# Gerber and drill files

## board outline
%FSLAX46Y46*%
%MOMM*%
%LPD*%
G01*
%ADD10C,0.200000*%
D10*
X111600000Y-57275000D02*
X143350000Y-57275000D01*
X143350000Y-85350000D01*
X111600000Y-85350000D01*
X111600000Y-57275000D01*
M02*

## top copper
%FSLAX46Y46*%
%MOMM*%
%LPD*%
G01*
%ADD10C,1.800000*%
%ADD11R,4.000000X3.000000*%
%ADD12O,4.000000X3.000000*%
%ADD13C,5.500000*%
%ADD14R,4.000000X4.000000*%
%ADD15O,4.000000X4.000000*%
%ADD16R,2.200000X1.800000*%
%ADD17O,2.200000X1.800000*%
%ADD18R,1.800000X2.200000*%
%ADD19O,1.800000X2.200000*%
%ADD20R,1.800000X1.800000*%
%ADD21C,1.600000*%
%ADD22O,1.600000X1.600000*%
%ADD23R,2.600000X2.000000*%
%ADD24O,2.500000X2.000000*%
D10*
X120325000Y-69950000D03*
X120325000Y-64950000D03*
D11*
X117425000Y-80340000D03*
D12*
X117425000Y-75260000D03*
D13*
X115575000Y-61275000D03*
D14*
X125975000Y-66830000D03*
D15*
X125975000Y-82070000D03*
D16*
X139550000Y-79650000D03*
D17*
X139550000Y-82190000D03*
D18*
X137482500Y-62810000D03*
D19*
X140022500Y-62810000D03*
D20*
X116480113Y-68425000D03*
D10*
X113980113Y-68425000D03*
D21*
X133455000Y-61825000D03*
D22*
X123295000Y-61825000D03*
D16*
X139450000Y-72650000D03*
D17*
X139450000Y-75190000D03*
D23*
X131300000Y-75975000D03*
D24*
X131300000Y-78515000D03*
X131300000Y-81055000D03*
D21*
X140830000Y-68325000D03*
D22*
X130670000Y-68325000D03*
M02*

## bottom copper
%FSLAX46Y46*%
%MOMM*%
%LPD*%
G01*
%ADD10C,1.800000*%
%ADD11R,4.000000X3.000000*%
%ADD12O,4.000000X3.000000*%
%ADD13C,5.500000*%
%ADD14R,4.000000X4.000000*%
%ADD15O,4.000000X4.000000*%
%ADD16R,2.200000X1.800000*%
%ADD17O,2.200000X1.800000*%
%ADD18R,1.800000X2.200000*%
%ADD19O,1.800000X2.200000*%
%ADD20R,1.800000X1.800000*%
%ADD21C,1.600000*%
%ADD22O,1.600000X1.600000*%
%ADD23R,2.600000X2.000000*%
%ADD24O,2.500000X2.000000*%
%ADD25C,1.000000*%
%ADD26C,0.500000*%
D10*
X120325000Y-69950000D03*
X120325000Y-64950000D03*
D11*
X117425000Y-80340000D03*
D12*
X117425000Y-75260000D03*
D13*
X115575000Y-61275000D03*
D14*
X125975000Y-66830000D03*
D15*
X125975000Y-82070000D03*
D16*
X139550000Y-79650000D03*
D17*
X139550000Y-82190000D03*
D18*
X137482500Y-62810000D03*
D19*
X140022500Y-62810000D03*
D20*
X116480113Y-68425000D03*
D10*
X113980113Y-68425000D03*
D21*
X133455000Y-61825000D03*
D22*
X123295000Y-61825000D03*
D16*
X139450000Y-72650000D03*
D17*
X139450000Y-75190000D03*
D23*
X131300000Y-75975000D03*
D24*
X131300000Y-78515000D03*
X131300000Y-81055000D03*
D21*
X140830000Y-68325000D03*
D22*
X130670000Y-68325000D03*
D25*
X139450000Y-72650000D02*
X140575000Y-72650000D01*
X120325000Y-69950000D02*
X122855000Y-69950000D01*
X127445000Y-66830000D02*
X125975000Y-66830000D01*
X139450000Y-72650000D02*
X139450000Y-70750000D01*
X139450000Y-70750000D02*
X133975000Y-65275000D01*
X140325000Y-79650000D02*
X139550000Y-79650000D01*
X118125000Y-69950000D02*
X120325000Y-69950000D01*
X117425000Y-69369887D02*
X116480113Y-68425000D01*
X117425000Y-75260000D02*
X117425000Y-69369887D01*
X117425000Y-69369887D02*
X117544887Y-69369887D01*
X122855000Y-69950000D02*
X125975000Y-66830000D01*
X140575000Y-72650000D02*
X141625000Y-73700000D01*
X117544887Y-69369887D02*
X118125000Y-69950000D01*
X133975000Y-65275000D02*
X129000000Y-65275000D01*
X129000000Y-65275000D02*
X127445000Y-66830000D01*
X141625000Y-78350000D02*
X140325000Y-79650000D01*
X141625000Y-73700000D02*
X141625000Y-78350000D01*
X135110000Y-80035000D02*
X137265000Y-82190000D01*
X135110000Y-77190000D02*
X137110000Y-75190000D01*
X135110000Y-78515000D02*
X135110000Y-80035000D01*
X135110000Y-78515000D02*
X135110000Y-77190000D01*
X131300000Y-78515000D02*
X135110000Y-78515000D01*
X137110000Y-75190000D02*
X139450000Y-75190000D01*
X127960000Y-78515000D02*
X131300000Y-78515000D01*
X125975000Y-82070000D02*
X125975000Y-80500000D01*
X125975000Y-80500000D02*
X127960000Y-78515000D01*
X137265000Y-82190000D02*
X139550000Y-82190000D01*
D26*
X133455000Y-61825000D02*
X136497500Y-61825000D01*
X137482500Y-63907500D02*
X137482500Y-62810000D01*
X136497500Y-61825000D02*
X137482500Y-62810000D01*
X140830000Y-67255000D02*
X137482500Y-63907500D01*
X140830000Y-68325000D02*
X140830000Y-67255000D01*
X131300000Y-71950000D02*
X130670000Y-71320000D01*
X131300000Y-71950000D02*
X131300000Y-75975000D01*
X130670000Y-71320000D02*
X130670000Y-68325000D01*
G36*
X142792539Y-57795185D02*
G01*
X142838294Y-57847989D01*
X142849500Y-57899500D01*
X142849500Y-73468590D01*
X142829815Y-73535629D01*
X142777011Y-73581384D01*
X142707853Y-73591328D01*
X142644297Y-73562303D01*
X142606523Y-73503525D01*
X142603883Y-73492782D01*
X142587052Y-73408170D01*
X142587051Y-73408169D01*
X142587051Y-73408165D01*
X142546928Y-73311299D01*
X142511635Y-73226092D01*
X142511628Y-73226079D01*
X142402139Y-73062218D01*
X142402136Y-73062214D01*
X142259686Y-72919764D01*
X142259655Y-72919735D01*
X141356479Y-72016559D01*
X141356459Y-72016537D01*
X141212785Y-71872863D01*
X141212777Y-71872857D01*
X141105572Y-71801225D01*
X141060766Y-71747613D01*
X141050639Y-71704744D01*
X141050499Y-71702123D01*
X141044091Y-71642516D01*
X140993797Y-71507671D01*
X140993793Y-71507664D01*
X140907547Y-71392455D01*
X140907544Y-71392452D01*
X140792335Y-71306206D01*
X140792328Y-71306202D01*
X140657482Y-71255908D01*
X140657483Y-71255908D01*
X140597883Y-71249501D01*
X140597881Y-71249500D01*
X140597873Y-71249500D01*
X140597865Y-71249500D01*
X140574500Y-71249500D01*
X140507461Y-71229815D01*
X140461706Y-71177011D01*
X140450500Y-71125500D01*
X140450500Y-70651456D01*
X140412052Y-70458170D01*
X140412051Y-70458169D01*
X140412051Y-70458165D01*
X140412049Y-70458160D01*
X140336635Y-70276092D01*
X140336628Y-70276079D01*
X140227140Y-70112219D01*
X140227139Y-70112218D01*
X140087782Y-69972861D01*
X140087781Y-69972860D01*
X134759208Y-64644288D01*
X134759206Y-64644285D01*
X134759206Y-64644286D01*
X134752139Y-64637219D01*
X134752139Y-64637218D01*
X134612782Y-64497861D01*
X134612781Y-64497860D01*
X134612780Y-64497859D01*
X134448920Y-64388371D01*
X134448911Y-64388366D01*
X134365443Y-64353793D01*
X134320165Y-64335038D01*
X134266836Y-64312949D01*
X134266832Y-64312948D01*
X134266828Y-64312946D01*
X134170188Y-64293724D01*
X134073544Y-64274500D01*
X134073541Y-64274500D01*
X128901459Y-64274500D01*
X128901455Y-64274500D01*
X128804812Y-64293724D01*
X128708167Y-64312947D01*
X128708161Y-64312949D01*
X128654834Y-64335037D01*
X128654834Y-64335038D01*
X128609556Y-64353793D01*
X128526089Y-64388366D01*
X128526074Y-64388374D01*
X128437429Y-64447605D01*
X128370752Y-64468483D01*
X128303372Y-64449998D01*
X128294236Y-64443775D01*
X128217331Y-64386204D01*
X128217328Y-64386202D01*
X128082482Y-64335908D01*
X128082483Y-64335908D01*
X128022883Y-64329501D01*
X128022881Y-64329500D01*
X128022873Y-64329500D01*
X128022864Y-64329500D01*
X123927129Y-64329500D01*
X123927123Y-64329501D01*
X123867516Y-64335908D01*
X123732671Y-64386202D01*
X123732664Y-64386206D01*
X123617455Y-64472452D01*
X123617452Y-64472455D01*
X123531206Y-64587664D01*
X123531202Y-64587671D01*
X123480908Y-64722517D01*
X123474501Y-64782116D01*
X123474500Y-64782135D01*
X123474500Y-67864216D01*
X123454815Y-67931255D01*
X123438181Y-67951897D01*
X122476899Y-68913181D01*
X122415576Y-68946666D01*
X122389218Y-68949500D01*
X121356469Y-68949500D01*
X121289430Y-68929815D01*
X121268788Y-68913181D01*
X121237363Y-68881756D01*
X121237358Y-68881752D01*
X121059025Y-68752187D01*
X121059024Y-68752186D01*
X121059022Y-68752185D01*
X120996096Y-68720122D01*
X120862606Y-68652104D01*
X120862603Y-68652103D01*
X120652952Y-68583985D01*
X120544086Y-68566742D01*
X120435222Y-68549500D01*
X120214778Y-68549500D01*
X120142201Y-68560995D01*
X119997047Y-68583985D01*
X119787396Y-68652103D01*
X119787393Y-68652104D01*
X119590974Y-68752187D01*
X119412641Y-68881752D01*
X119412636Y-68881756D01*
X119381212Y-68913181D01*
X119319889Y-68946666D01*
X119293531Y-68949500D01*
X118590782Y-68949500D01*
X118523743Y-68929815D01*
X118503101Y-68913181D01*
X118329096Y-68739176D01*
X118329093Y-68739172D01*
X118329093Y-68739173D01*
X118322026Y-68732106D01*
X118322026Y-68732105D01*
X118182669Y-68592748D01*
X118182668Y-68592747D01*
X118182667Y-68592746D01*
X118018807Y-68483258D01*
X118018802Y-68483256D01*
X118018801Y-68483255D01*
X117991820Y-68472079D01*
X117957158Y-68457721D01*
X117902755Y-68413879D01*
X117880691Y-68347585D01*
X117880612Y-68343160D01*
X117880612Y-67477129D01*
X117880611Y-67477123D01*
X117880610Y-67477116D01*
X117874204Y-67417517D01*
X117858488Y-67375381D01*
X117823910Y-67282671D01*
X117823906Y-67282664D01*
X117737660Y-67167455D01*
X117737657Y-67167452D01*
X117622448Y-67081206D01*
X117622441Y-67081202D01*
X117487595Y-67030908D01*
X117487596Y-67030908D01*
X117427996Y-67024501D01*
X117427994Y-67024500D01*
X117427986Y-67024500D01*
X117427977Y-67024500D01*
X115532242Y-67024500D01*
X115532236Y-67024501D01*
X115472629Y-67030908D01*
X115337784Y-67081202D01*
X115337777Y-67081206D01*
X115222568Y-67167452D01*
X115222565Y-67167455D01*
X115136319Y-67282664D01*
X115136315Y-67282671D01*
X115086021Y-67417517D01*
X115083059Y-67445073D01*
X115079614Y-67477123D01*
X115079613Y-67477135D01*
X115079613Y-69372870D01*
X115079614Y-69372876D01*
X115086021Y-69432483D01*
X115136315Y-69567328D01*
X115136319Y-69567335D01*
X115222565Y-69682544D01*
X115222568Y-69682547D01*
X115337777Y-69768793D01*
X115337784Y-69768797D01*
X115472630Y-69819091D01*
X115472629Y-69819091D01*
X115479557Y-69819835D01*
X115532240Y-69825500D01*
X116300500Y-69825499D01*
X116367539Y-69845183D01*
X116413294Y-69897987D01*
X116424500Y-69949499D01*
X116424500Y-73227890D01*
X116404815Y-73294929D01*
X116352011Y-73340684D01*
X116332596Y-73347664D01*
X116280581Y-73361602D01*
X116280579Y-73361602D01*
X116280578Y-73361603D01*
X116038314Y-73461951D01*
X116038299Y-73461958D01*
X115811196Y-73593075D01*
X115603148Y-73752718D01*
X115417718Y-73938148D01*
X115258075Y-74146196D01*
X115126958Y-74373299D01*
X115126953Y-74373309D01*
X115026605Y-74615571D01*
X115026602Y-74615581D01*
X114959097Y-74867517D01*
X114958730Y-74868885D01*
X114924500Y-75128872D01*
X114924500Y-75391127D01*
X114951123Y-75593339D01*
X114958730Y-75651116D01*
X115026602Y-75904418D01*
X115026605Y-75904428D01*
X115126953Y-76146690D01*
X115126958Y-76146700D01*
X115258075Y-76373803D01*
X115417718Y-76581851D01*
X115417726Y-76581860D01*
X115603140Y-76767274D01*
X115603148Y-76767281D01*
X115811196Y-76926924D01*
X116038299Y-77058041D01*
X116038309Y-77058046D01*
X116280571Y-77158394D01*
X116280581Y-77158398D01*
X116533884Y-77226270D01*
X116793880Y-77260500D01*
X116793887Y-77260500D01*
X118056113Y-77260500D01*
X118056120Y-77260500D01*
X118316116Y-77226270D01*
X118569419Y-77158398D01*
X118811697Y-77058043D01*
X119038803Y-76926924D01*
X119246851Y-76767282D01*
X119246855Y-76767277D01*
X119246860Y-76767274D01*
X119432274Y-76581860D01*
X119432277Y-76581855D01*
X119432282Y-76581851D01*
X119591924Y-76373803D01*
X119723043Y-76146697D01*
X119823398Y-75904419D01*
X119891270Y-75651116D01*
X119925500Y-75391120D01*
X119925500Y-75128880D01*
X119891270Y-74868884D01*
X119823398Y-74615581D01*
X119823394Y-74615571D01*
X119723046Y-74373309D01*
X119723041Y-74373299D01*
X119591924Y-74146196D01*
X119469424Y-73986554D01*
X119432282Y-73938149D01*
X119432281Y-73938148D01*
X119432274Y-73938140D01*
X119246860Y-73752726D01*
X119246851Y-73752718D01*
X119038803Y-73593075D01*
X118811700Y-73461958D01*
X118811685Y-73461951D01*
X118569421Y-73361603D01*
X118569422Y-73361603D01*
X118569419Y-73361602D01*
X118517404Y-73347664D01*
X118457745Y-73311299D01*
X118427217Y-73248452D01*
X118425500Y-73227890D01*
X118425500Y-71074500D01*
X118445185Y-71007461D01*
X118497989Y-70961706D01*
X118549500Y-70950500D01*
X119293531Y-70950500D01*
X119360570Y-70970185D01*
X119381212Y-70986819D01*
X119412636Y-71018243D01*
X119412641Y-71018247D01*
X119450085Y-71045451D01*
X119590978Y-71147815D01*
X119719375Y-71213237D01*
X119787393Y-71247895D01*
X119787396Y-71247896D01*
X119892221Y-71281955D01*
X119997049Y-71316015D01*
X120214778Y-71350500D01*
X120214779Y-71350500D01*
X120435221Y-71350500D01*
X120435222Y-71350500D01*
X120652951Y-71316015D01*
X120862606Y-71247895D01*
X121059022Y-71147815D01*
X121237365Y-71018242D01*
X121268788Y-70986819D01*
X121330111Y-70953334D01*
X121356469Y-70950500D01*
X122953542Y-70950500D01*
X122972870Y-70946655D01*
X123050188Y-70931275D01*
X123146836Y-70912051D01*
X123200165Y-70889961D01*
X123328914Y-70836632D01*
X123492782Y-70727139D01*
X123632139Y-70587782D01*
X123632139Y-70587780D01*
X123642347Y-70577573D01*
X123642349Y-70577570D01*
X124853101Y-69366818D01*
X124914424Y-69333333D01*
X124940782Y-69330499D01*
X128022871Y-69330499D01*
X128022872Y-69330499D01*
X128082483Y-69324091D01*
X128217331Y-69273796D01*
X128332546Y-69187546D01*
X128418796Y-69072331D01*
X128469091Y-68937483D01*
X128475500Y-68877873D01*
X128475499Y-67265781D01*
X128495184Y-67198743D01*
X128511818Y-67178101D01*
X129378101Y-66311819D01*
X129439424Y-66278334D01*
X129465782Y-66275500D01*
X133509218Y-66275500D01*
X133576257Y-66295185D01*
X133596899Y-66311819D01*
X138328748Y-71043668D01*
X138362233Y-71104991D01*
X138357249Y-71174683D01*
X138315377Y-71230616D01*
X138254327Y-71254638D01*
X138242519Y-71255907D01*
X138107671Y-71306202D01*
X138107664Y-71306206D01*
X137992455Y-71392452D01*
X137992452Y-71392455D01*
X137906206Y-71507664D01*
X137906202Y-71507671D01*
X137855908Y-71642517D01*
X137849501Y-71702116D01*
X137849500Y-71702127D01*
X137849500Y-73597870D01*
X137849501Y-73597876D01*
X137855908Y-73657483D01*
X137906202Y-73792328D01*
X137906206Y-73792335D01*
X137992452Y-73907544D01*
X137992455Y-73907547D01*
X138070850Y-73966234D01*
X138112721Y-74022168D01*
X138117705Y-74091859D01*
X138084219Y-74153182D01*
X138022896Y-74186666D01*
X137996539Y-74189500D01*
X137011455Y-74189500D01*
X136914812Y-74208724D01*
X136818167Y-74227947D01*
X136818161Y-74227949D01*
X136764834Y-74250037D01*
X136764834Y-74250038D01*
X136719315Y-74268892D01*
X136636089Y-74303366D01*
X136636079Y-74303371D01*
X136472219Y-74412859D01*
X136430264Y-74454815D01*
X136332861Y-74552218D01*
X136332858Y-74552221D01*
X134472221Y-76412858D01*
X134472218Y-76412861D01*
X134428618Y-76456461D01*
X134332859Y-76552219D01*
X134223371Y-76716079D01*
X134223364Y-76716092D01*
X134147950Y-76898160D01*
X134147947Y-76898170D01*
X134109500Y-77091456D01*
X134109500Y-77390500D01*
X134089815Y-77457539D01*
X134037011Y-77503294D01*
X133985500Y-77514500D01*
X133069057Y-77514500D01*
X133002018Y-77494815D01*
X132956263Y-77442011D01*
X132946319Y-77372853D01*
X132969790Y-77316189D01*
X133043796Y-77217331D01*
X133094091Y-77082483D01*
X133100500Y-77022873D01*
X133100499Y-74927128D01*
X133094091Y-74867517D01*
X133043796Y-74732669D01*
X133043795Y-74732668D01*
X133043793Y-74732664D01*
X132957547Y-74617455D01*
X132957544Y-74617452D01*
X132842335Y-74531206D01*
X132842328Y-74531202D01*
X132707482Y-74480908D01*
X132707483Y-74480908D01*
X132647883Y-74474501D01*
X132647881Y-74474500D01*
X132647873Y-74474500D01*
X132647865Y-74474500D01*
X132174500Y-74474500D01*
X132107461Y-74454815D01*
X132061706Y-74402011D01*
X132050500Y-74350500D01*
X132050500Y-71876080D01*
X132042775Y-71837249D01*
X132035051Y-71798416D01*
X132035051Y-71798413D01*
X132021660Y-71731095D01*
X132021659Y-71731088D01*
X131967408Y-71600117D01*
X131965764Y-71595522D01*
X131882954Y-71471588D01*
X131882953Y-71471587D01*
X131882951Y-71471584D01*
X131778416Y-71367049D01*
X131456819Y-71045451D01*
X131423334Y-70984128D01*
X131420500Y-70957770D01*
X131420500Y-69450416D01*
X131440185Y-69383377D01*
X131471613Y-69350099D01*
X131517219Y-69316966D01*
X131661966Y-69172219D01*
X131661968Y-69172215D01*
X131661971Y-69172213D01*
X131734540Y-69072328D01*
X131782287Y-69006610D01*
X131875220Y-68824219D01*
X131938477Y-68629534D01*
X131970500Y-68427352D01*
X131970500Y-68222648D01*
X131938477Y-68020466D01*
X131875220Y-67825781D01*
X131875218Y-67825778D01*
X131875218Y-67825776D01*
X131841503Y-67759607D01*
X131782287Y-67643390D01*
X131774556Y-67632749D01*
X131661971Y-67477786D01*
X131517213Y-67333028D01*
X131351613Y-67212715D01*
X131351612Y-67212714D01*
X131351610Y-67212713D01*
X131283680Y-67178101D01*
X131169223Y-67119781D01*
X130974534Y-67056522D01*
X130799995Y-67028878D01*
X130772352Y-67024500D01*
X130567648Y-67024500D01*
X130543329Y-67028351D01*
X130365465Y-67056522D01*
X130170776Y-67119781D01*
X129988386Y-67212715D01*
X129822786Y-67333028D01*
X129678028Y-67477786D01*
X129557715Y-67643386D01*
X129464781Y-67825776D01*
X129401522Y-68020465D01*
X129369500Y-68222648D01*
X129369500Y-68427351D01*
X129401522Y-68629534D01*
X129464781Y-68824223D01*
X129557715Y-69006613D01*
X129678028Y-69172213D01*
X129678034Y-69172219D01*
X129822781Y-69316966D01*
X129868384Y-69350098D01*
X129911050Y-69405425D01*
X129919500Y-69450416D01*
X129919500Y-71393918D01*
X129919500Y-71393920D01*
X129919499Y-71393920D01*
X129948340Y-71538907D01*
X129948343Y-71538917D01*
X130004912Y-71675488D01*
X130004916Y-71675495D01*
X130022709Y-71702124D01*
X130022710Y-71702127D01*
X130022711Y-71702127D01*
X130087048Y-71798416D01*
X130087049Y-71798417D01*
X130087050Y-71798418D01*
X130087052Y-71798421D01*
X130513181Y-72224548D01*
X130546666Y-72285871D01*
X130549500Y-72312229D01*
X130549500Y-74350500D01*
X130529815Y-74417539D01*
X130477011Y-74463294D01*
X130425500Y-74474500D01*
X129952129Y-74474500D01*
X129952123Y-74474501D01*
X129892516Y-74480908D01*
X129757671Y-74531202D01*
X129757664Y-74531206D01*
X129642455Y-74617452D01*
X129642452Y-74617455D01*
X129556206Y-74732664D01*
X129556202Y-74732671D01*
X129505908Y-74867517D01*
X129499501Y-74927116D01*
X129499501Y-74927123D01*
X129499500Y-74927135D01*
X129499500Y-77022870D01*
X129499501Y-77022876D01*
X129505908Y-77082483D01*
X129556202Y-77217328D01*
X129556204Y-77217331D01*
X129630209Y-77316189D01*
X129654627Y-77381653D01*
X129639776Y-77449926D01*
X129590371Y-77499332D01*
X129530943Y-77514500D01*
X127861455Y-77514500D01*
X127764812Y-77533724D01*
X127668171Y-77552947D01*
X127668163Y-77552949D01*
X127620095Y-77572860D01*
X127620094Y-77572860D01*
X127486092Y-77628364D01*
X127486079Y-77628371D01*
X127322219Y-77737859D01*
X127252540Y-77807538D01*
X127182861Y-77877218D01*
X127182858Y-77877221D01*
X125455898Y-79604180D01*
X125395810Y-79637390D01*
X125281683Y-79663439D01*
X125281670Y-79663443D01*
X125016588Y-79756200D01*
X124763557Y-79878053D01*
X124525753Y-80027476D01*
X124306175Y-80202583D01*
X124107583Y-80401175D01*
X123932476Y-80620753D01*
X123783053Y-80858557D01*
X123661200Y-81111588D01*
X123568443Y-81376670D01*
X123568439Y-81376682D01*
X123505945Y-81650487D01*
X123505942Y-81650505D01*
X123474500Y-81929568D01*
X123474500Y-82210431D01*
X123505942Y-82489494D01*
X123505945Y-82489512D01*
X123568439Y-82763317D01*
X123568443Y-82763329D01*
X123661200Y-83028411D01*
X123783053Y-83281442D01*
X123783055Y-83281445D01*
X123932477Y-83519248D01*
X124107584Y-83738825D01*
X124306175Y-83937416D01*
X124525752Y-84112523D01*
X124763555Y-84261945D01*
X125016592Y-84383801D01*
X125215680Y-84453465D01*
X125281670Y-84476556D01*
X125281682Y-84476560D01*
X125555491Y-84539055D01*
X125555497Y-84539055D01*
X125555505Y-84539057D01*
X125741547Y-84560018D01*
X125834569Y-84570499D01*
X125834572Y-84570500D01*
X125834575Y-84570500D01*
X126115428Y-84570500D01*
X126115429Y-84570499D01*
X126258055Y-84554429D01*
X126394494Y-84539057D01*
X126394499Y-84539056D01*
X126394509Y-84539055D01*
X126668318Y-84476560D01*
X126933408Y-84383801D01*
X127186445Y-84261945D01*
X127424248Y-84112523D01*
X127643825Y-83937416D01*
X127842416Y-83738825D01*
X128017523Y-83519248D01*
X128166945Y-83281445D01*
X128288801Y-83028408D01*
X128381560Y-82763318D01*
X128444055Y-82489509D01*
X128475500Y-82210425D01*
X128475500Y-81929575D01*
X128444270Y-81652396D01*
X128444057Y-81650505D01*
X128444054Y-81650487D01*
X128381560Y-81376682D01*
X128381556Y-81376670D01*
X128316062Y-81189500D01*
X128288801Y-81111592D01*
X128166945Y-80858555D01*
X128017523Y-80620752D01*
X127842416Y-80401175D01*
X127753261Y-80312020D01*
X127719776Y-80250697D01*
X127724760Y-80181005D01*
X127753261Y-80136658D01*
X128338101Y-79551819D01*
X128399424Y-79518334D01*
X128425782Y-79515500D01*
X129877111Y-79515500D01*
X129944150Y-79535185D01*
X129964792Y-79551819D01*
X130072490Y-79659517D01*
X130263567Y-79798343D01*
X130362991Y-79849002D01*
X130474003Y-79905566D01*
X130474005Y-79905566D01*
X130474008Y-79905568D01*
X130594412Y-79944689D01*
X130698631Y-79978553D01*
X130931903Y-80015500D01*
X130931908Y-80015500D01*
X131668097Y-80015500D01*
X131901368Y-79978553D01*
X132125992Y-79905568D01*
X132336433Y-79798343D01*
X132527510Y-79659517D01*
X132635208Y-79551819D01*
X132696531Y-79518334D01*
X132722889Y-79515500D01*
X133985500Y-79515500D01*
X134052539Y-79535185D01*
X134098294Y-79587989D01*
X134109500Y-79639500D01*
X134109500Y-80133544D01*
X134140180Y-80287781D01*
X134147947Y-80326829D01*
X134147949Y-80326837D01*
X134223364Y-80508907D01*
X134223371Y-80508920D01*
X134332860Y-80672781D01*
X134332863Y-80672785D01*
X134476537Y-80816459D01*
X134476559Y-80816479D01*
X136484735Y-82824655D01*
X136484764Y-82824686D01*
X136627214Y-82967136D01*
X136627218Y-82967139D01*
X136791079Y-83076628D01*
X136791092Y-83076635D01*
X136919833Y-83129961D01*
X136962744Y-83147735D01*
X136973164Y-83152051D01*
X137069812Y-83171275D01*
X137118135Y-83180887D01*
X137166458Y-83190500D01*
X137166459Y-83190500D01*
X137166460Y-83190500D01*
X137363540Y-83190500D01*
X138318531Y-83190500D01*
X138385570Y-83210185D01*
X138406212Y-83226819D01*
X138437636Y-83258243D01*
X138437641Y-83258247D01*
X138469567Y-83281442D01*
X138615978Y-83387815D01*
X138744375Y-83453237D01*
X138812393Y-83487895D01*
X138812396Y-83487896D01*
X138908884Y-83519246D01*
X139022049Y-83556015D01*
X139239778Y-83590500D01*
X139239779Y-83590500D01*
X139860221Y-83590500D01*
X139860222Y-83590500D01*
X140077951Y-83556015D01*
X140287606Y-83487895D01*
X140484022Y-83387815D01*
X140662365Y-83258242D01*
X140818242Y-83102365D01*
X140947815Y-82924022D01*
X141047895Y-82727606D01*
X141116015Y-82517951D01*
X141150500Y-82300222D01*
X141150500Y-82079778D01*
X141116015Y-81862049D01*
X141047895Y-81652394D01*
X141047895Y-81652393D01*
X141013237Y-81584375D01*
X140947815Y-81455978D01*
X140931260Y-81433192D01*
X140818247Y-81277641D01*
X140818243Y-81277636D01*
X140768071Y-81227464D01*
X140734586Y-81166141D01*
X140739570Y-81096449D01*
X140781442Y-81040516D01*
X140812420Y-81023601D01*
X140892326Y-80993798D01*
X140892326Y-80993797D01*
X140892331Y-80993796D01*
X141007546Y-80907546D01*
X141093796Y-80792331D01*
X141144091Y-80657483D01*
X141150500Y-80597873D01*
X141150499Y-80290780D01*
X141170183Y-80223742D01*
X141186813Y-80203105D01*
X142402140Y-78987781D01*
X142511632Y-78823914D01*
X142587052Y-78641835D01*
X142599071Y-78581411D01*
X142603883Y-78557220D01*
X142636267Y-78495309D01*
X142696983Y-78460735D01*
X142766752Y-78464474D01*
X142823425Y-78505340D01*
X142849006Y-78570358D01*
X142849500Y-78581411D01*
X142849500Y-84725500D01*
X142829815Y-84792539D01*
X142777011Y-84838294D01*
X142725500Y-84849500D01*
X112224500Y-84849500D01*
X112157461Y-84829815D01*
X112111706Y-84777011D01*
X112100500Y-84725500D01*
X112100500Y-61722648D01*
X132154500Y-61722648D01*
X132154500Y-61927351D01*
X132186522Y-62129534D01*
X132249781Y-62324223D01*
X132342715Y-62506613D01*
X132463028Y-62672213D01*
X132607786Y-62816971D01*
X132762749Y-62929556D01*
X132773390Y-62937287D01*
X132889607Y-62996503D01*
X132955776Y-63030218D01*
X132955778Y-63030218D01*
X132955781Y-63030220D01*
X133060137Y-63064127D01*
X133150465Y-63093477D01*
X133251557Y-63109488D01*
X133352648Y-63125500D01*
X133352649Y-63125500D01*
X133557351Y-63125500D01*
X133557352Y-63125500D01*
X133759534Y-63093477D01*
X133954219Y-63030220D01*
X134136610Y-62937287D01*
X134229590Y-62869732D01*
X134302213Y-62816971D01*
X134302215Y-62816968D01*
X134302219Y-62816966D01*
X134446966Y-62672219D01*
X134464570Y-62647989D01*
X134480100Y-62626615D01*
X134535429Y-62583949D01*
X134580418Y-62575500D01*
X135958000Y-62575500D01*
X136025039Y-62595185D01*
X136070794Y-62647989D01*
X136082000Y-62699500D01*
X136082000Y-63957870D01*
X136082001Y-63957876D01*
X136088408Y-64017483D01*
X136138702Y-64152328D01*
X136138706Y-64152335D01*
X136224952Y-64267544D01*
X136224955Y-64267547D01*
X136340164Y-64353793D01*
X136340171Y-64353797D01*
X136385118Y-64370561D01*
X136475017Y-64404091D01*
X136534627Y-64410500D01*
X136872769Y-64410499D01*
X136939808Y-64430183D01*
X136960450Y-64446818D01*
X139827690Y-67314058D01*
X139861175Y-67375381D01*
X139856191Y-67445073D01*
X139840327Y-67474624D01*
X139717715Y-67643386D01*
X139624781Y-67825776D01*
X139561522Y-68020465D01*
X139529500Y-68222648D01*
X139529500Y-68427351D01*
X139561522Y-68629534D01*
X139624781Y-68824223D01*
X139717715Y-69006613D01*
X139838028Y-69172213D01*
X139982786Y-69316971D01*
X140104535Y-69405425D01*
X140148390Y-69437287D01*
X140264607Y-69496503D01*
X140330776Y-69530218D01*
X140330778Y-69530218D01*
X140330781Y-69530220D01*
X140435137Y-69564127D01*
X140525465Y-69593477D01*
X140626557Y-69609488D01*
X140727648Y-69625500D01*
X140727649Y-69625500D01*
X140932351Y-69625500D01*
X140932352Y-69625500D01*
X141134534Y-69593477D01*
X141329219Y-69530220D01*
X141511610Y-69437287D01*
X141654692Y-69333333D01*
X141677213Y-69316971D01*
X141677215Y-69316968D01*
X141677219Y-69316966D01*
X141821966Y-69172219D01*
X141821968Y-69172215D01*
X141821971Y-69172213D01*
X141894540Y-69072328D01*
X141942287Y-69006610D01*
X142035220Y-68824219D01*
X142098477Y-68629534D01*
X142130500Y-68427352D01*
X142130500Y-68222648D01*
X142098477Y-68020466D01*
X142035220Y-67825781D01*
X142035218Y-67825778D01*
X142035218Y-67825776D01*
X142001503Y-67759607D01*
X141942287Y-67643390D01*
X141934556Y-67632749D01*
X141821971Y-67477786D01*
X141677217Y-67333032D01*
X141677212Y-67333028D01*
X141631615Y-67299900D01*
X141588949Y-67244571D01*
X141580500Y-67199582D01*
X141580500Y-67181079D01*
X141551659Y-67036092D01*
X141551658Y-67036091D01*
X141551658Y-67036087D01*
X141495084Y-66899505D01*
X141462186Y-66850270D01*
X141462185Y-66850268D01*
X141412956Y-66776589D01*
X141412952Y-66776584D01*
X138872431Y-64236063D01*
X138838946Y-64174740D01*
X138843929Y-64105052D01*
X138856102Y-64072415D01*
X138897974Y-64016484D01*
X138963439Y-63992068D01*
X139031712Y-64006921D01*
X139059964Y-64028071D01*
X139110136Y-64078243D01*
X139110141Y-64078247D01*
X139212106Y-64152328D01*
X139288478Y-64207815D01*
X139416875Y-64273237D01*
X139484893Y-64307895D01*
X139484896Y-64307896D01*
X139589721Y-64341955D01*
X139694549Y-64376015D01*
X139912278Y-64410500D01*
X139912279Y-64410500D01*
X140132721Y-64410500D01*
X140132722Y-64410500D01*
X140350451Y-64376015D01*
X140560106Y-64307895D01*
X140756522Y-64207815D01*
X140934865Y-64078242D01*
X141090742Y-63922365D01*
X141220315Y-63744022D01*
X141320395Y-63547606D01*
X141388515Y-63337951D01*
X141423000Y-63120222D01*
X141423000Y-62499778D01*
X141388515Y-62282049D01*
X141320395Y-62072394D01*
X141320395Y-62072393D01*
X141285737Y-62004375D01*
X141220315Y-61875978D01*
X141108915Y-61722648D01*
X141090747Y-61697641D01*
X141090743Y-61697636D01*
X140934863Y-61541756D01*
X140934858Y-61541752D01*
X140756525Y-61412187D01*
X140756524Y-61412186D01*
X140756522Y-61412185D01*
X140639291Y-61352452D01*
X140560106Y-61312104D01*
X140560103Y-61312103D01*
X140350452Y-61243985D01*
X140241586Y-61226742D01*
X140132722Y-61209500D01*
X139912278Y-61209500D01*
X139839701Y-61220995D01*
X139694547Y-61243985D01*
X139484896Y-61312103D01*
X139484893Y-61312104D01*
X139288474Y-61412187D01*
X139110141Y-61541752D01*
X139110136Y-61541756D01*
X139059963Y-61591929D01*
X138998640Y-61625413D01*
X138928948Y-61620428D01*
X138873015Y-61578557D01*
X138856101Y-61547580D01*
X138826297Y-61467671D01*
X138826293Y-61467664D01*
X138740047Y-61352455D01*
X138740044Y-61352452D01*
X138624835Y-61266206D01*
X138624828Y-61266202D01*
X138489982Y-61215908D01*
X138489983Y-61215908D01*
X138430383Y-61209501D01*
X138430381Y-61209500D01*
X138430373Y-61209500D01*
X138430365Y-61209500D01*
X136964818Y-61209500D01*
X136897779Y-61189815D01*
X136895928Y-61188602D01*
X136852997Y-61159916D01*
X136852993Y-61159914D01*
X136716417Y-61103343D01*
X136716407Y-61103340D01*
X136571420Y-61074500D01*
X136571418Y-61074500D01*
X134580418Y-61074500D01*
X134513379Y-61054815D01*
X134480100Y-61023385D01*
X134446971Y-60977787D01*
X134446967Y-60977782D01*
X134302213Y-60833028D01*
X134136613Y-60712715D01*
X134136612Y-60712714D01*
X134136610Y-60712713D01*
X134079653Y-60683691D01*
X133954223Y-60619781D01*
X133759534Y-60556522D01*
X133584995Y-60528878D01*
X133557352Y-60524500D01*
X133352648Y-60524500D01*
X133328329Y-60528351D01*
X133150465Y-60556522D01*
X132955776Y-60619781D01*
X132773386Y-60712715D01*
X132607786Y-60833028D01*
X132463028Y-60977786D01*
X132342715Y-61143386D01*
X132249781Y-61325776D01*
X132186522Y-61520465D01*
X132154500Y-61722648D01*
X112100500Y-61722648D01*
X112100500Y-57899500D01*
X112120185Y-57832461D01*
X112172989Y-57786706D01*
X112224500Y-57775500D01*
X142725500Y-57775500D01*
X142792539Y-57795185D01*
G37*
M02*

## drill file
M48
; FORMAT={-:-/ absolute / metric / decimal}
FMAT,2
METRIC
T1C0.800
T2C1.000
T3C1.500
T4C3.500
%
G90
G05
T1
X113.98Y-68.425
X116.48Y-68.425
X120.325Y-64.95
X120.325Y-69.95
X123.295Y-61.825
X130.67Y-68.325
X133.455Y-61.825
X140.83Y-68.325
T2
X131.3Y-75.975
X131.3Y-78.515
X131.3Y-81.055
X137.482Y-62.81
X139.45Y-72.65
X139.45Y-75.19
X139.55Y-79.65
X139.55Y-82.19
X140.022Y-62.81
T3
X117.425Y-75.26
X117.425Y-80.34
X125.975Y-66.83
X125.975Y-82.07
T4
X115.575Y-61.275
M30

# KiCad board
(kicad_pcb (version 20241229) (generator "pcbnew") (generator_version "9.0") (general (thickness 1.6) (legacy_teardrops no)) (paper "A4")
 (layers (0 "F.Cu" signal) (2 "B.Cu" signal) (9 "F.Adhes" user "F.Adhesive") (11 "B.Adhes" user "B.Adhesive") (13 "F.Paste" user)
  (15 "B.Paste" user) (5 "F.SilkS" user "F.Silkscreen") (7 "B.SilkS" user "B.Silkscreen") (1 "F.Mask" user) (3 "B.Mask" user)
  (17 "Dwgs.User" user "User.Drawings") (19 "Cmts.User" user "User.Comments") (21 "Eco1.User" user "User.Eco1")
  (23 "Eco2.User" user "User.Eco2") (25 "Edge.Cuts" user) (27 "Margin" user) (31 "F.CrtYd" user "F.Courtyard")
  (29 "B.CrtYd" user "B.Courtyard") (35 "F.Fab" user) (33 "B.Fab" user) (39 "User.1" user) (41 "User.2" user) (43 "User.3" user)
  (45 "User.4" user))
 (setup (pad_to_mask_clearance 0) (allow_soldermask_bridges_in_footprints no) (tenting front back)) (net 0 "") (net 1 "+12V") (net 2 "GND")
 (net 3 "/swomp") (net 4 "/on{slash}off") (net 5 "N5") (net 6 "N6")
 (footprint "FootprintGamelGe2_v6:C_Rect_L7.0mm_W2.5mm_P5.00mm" (layer "F.Cu") (at 120.325 69.95 90)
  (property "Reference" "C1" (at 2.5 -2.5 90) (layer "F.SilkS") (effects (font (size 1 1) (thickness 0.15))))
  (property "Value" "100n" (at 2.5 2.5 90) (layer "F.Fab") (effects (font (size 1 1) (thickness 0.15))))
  (pad "1" thru_hole circle (at 0 0 90) (size 1.8 1.8) (drill 0.8) (layers "*.Cu" "*.Mask") (remove_unused_layers no) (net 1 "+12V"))
  (pad "2" thru_hole circle (at 5 0 90) (size 1.8 1.8) (drill 0.8) (layers "*.Cu" "*.Mask") (remove_unused_layers no) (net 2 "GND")))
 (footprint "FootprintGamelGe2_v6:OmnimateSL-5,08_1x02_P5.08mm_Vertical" (layer "F.Cu") (at 117.425 80.34 90)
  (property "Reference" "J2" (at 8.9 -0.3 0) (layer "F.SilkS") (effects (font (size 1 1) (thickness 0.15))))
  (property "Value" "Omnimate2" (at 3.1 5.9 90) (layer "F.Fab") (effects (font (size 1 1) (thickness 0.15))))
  (pad "1" thru_hole rect (at 0 0 90) (size 3 4) (drill 1.5) (layers "*.Cu" "*.Mask") (remove_unused_layers no) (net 2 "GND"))
  (pad "2" thru_hole oval (at 5.08 0 90) (size 3 4) (drill 1.5) (layers "*.Cu" "*.Mask") (remove_unused_layers no) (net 1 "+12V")))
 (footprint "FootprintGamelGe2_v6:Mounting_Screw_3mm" (layer "F.Cu") (at 115.575 61.275)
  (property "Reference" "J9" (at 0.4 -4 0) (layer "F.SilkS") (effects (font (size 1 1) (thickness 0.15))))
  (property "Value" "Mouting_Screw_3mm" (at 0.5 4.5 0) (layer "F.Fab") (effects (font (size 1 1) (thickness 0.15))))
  (pad "1" thru_hole circle (at 0 0) (size 5.5 5.5) (drill 3.5) (layers "*.Cu" "*.Mask") (remove_unused_layers no) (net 2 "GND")))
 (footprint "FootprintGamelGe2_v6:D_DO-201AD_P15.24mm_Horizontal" (layer "F.Cu") (at 125.975 66.83 -90)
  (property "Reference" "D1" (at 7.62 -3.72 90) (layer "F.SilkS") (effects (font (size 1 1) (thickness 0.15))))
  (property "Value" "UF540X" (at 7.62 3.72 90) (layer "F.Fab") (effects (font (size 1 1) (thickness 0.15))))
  (pad "1" thru_hole rect (at 0 0 270) (size 4 4) (drill 1.5) (layers "*.Cu" "*.Mask") (remove_unused_layers no) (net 1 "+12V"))
  (pad "2" thru_hole oval (at 15.24 0 270) (size 4 4) (drill 1.5) (layers "*.Cu" "*.Mask") (remove_unused_layers no) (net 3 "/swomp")))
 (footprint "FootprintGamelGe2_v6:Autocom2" (layer "F.Cu") (at 139.55 79.65)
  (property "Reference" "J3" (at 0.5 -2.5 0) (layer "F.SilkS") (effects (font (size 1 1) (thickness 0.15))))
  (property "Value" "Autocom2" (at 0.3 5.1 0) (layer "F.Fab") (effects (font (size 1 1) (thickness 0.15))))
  (pad "1" thru_hole rect (at 0 0) (size 2.2 1.8) (drill 1) (layers "*.Cu" "*.Mask") (remove_unused_layers no) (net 1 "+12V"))
  (pad "2" thru_hole oval (at 0 2.54) (size 2.2 1.8) (drill 1) (layers "*.Cu" "*.Mask") (remove_unused_layers no) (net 3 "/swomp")))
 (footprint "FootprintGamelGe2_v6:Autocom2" (layer "F.Cu") (at 137.4825 62.81 90)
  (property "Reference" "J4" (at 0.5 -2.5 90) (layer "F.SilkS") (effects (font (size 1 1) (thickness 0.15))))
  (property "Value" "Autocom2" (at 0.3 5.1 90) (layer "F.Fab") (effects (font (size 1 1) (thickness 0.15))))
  (pad "1" thru_hole rect (at 0 0 90) (size 2.2 1.8) (drill 1) (layers "*.Cu" "*.Mask") (remove_unused_layers no) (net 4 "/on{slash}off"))
  (pad "2" thru_hole oval (at 0 2.54 90) (size 2.2 1.8) (drill 1) (layers "*.Cu" "*.Mask") (remove_unused_layers no) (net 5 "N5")))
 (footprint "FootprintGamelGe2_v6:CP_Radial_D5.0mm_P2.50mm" (layer "F.Cu") (at 116.480113 68.425 180)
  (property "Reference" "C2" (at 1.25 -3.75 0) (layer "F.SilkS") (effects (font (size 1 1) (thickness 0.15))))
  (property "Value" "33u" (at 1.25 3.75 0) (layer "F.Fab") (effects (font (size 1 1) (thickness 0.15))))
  (pad "1" thru_hole rect (at 0 0 180) (size 1.8 1.8) (drill 0.8) (layers "*.Cu" "*.Mask") (remove_unused_layers no) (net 1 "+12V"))
  (pad "2" thru_hole circle (at 2.5 0 180) (size 1.8 1.8) (drill 0.8) (layers "*.Cu" "*.Mask") (remove_unused_layers no) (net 2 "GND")))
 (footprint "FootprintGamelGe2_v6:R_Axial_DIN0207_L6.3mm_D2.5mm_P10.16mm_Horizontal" (layer "F.Cu") (at 133.455 61.825 180)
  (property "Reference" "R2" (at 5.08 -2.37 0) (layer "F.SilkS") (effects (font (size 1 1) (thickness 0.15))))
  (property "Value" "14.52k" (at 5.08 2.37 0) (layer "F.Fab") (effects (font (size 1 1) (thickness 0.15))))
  (pad "1" thru_hole circle (at 0 0 180) (size 1.6 1.6) (drill 0.8) (layers "*.Cu" "*.Mask") (remove_unused_layers no)
   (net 4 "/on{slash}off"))
  (pad "2" thru_hole oval (at 10.16 0 180) (size 1.6 1.6) (drill 0.8) (layers "*.Cu" "*.Mask") (remove_unused_layers no) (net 2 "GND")))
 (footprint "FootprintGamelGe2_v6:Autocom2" (layer "F.Cu") (at 139.45 72.65)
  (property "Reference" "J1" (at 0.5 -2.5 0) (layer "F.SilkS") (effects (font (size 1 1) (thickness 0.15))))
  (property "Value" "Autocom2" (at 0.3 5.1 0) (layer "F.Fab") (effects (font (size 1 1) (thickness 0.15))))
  (pad "1" thru_hole rect (at 0 0) (size 2.2 1.8) (drill 1) (layers "*.Cu" "*.Mask") (remove_unused_layers no) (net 1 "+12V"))
  (pad "2" thru_hole oval (at 0 2.54) (size 2.2 1.8) (drill 1) (layers "*.Cu" "*.Mask") (remove_unused_layers no) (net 3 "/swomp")))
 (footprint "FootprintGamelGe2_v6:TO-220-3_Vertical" (layer "F.Cu") (at 131.3 75.975 -90)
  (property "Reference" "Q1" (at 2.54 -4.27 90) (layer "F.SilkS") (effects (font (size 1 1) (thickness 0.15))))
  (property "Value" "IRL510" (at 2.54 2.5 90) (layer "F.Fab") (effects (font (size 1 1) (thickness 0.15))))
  (pad "1" thru_hole rect (at 0 0 270) (size 2 2.6) (drill 1) (layers "*.Cu" "*.Mask") (remove_unused_layers no) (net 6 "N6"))
  (pad "2" thru_hole oval (at 2.54 0 270) (size 2 2.5) (drill 1) (layers "*.Cu" "*.Mask") (remove_unused_layers no) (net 3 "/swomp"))
  (pad "3" thru_hole oval (at 5.08 0 270) (size 2 2.5) (drill 1) (layers "*.Cu" "*.Mask") (remove_unused_layers no) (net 2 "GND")))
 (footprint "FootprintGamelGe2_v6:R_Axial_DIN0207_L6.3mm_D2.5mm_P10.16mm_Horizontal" (layer "F.Cu") (at 140.83 68.325 180)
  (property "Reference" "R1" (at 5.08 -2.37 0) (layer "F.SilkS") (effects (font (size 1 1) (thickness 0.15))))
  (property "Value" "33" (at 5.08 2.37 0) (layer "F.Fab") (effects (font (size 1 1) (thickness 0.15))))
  (pad "1" thru_hole circle (at 0 0 180) (size 1.6 1.6) (drill 0.8) (layers "*.Cu" "*.Mask") (remove_unused_layers no)
   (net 4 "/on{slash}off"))
  (pad "2" thru_hole oval (at 10.16 0 180) (size 1.6 1.6) (drill 0.8) (layers "*.Cu" "*.Mask") (remove_unused_layers no) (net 6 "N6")))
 (gr_rect (start 111.6 57.275) (end 143.35 85.35) (stroke (width 0.2) (type solid)) (fill no) (layer "Edge.Cuts"))
 (segment (start 139.45 72.65) (end 140.575 72.65) (width 1) (layer "B.Cu") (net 1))
 (segment (start 120.325 69.95) (end 122.855 69.95) (width 1) (layer "B.Cu") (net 1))
 (segment (start 127.445 66.83) (end 125.975 66.83) (width 1) (layer "B.Cu") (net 1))
 (segment (start 139.45 72.65) (end 139.45 70.75) (width 1) (layer "B.Cu") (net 1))
 (segment (start 139.45 70.75) (end 133.975 65.275) (width 1) (layer "B.Cu") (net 1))
 (segment (start 140.325 79.65) (end 139.55 79.65) (width 1) (layer "B.Cu") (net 1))
 (segment (start 118.125 69.95) (end 120.325 69.95) (width 1) (layer "B.Cu") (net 1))
 (segment (start 117.425 69.369887) (end 116.480113 68.425) (width 1) (layer "B.Cu") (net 1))
 (segment (start 117.425 75.26) (end 117.425 69.369887) (width 1) (layer "B.Cu") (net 1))
 (segment (start 117.425 69.369887) (end 117.544887 69.369887) (width 1) (layer "B.Cu") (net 1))
 (segment (start 122.855 69.95) (end 125.975 66.83) (width 1) (layer "B.Cu") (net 1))
 (segment (start 140.575 72.65) (end 141.625 73.7) (width 1) (layer "B.Cu") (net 1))
 (segment (start 117.544887 69.369887) (end 118.125 69.95) (width 1) (layer "B.Cu") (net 1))
 (segment (start 133.975 65.275) (end 129 65.275) (width 1) (layer "B.Cu") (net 1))
 (segment (start 129 65.275) (end 127.445 66.83) (width 1) (layer "B.Cu") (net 1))
 (segment (start 141.625 78.35) (end 140.325 79.65) (width 1) (layer "B.Cu") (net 1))
 (segment (start 141.625 73.7) (end 141.625 78.35) (width 1) (layer "B.Cu") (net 1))
 (segment (start 135.11 80.035) (end 137.265 82.19) (width 1) (layer "B.Cu") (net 3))
 (segment (start 135.11 77.19) (end 137.11 75.19) (width 1) (layer "B.Cu") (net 3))
 (segment (start 135.11 78.515) (end 135.11 80.035) (width 1) (layer "B.Cu") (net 3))
 (segment (start 135.11 78.515) (end 135.11 77.19) (width 1) (layer "B.Cu") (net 3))
 (segment (start 131.3 78.515) (end 135.11 78.515) (width 1) (layer "B.Cu") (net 3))
 (segment (start 137.11 75.19) (end 139.45 75.19) (width 1) (layer "B.Cu") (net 3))
 (segment (start 127.96 78.515) (end 131.3 78.515) (width 1) (layer "B.Cu") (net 3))
 (segment (start 125.975 82.07) (end 125.975 80.5) (width 1) (layer "B.Cu") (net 3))
 (segment (start 125.975 80.5) (end 127.96 78.515) (width 1) (layer "B.Cu") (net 3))
 (segment (start 137.265 82.19) (end 139.55 82.19) (width 1) (layer "B.Cu") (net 3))
 (segment (start 133.455 61.825) (end 136.4975 61.825) (width 0.5) (layer "B.Cu") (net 4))
 (segment (start 137.4825 63.9075) (end 137.4825 62.81) (width 0.5) (layer "B.Cu") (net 4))
 (segment (start 136.4975 61.825) (end 137.4825 62.81) (width 0.5) (layer "B.Cu") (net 4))
 (segment (start 140.83 67.255) (end 137.4825 63.9075) (width 0.5) (layer "B.Cu") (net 4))
 (segment (start 140.83 68.325) (end 140.83 67.255) (width 0.5) (layer "B.Cu") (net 4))
 (segment (start 131.3 71.95) (end 130.67 71.32) (width 0.5) (layer "B.Cu") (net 6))
 (segment (start 131.3 71.95) (end 131.3 75.975) (width 0.5) (layer "B.Cu") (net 6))
 (segment (start 130.67 71.32) (end 130.67 68.325) (width 0.5) (layer "B.Cu") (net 6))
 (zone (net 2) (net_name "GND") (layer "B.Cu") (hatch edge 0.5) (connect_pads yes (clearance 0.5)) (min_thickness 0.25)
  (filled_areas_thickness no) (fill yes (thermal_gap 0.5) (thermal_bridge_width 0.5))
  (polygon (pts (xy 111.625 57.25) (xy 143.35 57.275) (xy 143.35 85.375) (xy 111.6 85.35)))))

